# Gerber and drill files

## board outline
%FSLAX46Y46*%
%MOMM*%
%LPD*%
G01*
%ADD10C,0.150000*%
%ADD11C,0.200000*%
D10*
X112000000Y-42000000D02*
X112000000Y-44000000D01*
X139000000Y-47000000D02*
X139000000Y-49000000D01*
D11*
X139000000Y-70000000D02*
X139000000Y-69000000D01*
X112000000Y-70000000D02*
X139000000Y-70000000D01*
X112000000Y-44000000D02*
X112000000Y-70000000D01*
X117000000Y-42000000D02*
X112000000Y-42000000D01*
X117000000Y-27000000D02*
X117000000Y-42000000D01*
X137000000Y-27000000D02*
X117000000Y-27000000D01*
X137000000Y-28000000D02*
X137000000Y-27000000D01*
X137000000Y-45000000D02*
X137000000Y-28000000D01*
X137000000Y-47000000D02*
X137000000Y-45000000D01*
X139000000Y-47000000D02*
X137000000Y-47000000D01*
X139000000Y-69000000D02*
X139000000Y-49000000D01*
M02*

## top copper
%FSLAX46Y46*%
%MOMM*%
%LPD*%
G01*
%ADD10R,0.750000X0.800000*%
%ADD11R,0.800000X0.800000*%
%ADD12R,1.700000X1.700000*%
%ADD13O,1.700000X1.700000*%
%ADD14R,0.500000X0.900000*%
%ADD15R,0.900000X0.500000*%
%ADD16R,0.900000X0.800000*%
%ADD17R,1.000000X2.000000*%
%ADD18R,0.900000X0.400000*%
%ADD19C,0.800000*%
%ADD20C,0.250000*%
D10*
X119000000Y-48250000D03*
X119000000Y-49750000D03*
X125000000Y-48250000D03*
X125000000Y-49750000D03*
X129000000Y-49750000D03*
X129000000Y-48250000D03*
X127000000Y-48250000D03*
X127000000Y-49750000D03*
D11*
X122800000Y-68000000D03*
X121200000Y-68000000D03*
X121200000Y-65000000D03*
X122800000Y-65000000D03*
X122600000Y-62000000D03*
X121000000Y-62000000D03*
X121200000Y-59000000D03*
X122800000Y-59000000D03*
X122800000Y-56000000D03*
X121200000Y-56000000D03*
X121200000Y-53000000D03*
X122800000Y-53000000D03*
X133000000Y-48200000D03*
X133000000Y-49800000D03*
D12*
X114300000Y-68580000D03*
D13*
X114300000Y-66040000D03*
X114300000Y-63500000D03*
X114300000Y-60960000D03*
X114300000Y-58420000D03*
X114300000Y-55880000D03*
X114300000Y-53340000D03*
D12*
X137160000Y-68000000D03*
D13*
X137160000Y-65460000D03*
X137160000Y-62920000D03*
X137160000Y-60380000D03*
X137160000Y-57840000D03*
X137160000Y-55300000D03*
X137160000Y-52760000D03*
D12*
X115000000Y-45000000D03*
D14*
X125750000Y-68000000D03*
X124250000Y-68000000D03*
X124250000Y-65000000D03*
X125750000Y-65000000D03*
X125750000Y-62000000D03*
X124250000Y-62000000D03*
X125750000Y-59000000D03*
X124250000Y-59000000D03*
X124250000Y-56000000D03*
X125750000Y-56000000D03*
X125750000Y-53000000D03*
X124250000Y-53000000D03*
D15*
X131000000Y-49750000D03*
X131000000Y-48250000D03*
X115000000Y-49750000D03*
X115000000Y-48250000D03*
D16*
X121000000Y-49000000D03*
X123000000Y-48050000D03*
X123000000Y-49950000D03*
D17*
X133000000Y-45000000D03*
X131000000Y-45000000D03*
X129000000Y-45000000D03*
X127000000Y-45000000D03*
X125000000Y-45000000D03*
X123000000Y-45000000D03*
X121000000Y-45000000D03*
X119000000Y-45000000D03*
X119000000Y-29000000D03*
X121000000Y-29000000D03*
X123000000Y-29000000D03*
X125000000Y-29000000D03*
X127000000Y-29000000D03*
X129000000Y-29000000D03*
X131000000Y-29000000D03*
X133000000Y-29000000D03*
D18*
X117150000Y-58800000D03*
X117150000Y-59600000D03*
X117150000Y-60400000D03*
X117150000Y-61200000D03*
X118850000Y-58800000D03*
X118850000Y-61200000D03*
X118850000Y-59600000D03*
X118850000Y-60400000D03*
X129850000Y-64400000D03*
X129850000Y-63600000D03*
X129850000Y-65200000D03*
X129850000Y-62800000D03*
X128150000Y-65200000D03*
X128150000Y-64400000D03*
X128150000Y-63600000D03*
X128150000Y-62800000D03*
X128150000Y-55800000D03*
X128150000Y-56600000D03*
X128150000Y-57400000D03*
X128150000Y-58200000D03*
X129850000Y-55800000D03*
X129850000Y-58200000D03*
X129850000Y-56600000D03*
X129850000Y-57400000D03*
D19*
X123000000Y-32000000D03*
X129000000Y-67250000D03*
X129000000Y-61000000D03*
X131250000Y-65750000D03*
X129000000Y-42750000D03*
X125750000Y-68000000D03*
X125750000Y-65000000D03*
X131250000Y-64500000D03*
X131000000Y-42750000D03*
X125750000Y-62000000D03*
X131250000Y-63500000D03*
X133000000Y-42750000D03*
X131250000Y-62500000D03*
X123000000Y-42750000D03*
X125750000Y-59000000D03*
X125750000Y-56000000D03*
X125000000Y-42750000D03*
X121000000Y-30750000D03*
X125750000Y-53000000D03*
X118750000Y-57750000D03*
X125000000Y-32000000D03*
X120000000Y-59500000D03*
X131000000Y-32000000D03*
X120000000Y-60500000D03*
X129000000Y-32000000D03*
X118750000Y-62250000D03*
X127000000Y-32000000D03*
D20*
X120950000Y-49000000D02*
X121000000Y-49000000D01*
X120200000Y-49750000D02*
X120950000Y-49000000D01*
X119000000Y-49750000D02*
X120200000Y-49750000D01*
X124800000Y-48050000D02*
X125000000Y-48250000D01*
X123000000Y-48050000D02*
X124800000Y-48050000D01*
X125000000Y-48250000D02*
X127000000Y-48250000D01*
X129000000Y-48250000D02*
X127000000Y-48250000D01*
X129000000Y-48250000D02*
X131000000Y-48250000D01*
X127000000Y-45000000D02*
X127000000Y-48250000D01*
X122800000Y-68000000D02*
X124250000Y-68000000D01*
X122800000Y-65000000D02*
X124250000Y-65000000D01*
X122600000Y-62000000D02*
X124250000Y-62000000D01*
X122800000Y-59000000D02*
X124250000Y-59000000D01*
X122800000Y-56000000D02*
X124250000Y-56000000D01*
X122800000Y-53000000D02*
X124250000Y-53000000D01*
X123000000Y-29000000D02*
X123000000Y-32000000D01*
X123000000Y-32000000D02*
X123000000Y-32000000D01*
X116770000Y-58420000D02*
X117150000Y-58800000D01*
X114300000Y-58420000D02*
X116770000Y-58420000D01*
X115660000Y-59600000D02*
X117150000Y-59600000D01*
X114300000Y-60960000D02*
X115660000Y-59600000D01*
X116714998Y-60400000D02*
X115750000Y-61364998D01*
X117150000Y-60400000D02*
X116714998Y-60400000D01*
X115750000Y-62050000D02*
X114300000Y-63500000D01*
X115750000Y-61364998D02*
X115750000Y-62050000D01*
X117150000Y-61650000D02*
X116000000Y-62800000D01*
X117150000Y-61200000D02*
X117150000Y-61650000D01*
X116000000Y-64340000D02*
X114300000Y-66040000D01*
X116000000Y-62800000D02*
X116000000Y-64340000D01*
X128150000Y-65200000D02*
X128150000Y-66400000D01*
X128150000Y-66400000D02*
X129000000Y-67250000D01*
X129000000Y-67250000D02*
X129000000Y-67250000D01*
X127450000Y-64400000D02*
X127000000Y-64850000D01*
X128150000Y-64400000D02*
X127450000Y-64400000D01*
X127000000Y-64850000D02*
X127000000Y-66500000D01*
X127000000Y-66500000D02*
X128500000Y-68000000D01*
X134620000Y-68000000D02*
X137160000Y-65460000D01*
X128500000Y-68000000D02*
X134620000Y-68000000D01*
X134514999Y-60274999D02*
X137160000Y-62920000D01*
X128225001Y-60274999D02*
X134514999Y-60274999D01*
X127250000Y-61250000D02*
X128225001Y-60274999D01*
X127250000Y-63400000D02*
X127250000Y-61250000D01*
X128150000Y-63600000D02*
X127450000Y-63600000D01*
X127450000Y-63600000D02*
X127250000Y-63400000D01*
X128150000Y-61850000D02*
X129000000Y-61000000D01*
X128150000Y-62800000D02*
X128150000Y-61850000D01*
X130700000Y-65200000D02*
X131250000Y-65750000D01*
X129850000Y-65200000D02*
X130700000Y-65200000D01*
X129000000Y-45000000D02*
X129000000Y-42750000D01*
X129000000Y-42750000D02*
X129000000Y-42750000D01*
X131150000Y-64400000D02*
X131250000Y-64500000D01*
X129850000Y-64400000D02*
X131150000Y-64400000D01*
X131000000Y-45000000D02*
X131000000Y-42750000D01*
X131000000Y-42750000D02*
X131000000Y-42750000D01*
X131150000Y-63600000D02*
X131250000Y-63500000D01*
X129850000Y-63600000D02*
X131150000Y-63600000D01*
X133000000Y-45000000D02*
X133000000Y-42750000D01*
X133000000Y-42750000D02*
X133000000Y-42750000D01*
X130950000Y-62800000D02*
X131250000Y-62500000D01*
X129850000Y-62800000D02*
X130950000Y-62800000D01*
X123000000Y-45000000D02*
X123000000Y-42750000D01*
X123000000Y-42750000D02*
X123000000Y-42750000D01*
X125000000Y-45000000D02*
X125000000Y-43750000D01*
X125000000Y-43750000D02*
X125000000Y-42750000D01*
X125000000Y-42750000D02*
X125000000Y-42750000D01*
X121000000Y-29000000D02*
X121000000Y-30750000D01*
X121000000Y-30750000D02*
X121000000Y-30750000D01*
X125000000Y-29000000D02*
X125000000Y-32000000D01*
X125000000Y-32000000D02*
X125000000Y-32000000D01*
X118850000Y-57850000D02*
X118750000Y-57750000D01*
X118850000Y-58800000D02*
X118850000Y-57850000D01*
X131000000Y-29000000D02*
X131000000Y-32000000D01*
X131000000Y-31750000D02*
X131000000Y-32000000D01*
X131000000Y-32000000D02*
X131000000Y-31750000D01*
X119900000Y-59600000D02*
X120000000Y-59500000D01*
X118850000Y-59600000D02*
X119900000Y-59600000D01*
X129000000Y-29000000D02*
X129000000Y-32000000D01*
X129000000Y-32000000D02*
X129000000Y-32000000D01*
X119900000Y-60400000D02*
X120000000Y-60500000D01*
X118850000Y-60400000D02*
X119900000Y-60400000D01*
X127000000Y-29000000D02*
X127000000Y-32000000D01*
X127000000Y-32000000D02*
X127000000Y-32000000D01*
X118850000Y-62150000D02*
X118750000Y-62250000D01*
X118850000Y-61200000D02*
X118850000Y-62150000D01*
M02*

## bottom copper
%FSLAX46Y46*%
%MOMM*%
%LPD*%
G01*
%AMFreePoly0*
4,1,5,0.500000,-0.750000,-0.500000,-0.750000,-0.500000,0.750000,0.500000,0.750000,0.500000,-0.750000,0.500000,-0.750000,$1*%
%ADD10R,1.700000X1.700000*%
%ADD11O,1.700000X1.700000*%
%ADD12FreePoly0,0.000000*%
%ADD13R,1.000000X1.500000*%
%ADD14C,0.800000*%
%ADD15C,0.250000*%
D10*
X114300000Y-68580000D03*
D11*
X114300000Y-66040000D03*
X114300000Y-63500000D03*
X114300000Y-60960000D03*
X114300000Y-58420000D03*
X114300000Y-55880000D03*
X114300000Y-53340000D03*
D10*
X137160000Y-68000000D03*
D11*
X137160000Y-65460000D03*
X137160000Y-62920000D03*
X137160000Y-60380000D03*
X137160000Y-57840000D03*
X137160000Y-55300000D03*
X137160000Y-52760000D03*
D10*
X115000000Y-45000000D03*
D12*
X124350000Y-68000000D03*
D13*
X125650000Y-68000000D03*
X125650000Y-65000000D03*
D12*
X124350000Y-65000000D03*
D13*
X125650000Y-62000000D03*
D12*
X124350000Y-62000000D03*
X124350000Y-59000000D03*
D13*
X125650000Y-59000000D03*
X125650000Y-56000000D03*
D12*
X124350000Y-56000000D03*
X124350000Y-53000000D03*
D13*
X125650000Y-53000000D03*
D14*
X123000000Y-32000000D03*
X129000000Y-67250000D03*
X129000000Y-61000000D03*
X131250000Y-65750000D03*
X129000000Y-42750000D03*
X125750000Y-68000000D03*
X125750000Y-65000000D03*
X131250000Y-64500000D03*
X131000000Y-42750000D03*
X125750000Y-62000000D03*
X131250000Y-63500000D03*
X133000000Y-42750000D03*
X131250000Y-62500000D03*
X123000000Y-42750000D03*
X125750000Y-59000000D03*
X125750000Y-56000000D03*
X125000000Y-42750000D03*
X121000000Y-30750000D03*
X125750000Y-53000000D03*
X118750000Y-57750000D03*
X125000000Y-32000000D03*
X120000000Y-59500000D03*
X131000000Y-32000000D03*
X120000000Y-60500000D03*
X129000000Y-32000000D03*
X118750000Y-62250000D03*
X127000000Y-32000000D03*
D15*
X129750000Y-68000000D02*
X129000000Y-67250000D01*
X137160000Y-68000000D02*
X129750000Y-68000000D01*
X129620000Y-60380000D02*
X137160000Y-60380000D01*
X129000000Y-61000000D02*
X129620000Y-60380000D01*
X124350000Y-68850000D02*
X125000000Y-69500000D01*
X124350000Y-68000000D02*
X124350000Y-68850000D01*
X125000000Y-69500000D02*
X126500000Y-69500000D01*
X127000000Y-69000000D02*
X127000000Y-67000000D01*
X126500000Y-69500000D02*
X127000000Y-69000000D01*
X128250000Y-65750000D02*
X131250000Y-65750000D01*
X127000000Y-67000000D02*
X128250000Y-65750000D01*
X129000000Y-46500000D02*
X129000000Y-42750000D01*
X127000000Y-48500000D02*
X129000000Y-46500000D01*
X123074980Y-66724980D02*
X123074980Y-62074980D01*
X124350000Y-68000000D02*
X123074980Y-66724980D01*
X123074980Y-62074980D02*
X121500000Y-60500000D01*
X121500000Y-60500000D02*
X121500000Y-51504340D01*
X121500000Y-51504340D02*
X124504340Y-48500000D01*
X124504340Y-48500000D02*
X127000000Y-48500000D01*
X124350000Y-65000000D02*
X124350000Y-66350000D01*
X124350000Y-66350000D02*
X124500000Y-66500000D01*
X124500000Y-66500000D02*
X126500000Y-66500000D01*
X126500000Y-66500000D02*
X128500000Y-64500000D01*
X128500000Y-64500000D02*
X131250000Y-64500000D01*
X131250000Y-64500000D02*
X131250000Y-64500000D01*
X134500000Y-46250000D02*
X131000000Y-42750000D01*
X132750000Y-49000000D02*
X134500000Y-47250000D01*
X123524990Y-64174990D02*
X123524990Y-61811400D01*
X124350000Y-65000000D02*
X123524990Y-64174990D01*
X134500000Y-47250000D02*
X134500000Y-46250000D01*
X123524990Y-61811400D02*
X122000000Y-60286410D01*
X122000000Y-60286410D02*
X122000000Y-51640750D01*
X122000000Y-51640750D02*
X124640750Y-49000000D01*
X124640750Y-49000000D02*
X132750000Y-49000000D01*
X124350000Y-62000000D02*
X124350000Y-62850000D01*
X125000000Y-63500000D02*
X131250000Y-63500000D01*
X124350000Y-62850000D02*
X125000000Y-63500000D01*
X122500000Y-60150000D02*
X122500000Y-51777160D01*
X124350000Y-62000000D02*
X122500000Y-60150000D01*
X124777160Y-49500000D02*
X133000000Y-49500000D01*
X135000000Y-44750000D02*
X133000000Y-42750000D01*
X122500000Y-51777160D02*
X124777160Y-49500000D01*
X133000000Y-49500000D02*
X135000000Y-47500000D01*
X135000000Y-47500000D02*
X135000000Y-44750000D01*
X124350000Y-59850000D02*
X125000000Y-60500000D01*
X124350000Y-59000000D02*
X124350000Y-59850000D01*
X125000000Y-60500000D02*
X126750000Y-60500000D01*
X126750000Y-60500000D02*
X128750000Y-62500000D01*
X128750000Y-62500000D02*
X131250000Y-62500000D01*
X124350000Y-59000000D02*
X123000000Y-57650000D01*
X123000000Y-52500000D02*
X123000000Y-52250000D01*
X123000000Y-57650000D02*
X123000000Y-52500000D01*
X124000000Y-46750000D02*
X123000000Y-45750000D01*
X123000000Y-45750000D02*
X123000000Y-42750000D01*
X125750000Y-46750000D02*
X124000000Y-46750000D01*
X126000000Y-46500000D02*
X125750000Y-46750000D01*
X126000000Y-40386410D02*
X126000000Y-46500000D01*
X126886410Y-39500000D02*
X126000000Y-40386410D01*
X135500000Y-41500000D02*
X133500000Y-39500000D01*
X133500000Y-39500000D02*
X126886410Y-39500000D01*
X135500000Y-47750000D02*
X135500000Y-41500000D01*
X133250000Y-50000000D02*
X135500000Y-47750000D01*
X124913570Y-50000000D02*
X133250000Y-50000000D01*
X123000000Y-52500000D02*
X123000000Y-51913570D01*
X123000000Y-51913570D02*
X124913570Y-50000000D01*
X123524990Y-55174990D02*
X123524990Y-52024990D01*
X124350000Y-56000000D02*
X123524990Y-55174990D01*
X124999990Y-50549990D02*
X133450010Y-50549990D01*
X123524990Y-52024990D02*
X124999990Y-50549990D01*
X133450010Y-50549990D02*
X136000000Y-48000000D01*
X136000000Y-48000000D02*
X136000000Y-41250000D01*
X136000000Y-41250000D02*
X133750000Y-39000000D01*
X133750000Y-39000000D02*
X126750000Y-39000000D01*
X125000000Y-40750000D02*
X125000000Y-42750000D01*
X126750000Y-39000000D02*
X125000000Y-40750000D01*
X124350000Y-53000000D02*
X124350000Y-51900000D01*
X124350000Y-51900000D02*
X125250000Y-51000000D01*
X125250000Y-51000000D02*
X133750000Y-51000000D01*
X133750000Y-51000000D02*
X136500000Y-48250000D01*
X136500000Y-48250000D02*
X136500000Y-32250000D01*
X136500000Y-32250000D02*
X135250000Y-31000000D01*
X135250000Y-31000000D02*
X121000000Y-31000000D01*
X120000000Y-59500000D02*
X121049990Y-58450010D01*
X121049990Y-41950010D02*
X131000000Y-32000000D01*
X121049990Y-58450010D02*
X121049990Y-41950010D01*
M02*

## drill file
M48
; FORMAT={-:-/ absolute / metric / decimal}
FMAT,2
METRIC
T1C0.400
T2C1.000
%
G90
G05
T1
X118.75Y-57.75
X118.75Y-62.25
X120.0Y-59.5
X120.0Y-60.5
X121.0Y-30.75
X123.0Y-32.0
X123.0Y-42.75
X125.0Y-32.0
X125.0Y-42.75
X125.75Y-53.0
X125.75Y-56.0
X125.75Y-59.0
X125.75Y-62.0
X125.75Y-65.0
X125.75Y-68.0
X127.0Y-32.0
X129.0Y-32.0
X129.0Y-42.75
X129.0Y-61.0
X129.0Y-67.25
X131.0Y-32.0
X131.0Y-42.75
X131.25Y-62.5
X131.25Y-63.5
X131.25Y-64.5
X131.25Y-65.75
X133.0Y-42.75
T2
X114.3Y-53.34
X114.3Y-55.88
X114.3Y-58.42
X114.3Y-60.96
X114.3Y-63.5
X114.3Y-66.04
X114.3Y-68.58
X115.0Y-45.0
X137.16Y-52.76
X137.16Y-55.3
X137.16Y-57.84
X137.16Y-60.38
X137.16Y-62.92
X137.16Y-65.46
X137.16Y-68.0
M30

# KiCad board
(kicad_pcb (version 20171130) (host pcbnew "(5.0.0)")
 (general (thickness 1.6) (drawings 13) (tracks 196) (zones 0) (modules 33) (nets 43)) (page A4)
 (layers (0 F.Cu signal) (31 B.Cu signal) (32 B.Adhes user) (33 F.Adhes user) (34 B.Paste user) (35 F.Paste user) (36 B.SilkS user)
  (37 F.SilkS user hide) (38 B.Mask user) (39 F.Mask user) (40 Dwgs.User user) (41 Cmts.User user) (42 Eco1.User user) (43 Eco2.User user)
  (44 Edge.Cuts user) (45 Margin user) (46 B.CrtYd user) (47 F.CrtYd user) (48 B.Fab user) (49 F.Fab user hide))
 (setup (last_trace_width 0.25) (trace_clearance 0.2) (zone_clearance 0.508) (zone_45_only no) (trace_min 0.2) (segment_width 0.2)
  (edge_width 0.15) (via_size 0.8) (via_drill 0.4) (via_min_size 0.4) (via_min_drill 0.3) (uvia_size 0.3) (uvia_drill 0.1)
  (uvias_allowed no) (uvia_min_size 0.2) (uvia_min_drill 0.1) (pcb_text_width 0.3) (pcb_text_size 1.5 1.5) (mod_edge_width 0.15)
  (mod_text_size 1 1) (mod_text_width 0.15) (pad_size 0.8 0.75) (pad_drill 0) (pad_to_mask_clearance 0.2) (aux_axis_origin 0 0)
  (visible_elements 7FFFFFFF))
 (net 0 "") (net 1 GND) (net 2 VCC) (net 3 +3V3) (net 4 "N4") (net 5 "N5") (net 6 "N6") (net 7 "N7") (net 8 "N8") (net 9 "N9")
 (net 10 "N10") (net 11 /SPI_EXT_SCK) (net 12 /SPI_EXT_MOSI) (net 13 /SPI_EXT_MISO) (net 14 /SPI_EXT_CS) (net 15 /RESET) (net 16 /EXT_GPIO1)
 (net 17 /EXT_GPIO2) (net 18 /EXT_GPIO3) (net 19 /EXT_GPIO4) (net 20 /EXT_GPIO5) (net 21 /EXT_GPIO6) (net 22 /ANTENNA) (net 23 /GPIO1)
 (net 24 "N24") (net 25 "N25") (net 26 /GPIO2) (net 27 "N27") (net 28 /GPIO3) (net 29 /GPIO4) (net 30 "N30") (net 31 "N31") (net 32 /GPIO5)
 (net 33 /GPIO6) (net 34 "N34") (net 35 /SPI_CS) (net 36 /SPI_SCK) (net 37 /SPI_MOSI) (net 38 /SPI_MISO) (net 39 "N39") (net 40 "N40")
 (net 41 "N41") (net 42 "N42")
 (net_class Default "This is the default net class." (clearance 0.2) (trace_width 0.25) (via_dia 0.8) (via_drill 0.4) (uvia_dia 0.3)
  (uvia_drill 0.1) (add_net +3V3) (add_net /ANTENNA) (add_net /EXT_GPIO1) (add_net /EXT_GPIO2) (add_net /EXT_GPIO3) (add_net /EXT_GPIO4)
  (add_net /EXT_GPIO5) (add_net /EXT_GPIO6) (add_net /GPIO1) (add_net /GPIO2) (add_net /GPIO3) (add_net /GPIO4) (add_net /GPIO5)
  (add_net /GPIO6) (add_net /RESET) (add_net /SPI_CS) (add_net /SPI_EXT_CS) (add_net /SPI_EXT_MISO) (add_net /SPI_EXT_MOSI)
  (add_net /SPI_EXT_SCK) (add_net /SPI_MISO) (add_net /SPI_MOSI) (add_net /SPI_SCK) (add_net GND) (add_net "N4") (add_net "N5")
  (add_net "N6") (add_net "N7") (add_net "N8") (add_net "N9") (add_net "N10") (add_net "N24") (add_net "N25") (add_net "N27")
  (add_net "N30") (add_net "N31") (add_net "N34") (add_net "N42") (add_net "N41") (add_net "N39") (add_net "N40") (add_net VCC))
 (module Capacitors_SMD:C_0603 (layer F.Cu) (at 119 49 90)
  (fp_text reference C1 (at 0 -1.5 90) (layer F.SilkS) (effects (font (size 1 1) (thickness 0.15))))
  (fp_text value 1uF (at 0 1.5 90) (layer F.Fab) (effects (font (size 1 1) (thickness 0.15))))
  (pad 2 smd rect (at 0.75 0 90) (size 0.8 0.75) (layers F.Cu F.Paste F.Mask) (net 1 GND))
  (pad 1 smd rect (at -0.75 0 90) (size 0.8 0.75) (layers F.Cu F.Paste F.Mask) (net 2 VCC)))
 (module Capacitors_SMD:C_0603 (layer F.Cu) (at 125 49 270)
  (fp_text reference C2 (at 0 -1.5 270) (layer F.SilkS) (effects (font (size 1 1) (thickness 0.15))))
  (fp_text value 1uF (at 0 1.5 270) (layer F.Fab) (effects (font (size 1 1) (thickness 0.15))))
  (pad 1 smd rect (at -0.75 0 270) (size 0.8 0.75) (layers F.Cu F.Paste F.Mask) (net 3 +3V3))
  (pad 2 smd rect (at 0.75 0 270) (size 0.8 0.75) (layers F.Cu F.Paste F.Mask) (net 1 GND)))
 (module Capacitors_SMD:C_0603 (layer F.Cu) (at 129 49 270)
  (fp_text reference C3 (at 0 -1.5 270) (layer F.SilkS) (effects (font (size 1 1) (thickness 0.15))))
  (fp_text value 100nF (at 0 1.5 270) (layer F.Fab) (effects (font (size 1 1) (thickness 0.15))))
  (pad 2 smd rect (at 0.75 0 270) (size 0.8 0.75) (layers F.Cu F.Paste F.Mask) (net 1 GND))
  (pad 1 smd rect (at -0.75 0 270) (size 0.8 0.75) (layers F.Cu F.Paste F.Mask) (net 3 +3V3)))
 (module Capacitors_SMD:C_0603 (layer F.Cu) (at 127 49 270)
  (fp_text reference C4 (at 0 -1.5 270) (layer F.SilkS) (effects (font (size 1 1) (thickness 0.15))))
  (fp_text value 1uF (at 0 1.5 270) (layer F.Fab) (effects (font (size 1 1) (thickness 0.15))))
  (pad 1 smd rect (at -0.75 0 270) (size 0.8 0.75) (layers F.Cu F.Paste F.Mask) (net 3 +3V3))
  (pad 2 smd rect (at 0.75 0 270) (size 0.8 0.75) (layers F.Cu F.Paste F.Mask) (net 1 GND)))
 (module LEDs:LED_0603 (layer F.Cu) (at 122 68)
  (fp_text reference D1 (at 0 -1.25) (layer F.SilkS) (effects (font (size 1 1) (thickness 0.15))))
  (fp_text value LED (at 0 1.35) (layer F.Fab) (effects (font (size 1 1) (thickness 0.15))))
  (pad 2 smd rect (at 0.8 0 180) (size 0.8 0.8) (layers F.Cu F.Paste F.Mask) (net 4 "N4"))
  (pad 1 smd rect (at -0.8 0 180) (size 0.8 0.8) (layers F.Cu F.Paste F.Mask) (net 1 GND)))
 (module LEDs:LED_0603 (layer F.Cu) (at 122 65)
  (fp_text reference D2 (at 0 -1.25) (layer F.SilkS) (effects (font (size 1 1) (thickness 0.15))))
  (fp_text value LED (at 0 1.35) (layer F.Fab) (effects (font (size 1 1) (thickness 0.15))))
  (pad 1 smd rect (at -0.8 0 180) (size 0.8 0.8) (layers F.Cu F.Paste F.Mask) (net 1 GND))
  (pad 2 smd rect (at 0.8 0 180) (size 0.8 0.8) (layers F.Cu F.Paste F.Mask) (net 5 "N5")))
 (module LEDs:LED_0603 (layer F.Cu) (at 121.8 62)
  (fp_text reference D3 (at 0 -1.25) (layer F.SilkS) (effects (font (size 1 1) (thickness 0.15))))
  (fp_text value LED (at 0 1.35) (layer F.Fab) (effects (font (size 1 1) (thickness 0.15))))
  (pad 2 smd rect (at 0.8 0 180) (size 0.8 0.8) (layers F.Cu F.Paste F.Mask) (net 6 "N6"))
  (pad 1 smd rect (at -0.8 0 180) (size 0.8 0.8) (layers F.Cu F.Paste F.Mask) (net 1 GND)))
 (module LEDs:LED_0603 (layer F.Cu) (at 122 59)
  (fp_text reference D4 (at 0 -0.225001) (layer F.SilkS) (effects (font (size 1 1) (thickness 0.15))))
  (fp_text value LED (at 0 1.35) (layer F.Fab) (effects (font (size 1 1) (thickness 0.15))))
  (pad 1 smd rect (at -0.8 0 180) (size 0.8 0.8) (layers F.Cu F.Paste F.Mask) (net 1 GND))
  (pad 2 smd rect (at 0.8 0 180) (size 0.8 0.8) (layers F.Cu F.Paste F.Mask) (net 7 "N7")))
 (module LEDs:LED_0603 (layer F.Cu) (at 122 56)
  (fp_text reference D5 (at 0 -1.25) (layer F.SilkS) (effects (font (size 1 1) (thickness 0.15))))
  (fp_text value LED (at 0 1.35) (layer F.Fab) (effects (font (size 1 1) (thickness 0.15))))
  (pad 2 smd rect (at 0.8 0 180) (size 0.8 0.8) (layers F.Cu F.Paste F.Mask) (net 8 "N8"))
  (pad 1 smd rect (at -0.8 0 180) (size 0.8 0.8) (layers F.Cu F.Paste F.Mask) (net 1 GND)))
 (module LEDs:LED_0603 (layer F.Cu) (at 122 53)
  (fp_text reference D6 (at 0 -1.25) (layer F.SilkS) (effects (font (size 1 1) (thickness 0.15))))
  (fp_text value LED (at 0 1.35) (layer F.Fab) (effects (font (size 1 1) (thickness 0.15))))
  (pad 1 smd rect (at -0.8 0 180) (size 0.8 0.8) (layers F.Cu F.Paste F.Mask) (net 1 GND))
  (pad 2 smd rect (at 0.8 0 180) (size 0.8 0.8) (layers F.Cu F.Paste F.Mask) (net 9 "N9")))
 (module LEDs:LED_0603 (layer F.Cu) (at 133 49 270)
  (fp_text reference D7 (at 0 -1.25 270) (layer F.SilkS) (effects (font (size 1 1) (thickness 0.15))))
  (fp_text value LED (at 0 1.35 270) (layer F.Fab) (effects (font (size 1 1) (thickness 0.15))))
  (pad 1 smd rect (at -0.8 0 90) (size 0.8 0.8) (layers F.Cu F.Paste F.Mask) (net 1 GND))
  (pad 2 smd rect (at 0.8 0 90) (size 0.8 0.8) (layers F.Cu F.Paste F.Mask) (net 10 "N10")))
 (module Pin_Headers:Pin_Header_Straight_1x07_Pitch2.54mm (layer F.Cu) (at 114.3 68.58 180)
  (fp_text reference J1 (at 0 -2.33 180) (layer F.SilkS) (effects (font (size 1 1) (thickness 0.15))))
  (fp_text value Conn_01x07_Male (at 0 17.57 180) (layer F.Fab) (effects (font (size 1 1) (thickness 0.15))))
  (pad 1 thru_hole rect (at 0 0 180) (size 1.7 1.7) (drill 1) (layers *.Cu *.Mask) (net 2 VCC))
  (pad 2 thru_hole oval (at 0 2.54 180) (size 1.7 1.7) (drill 1) (layers *.Cu *.Mask) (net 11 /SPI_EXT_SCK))
  (pad 3 thru_hole oval (at 0 5.08 180) (size 1.7 1.7) (drill 1) (layers *.Cu *.Mask) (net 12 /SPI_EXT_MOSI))
  (pad 4 thru_hole oval (at 0 7.62 180) (size 1.7 1.7) (drill 1) (layers *.Cu *.Mask) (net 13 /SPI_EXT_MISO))
  (pad 5 thru_hole oval (at 0 10.16 180) (size 1.7 1.7) (drill 1) (layers *.Cu *.Mask) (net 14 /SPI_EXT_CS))
  (pad 6 thru_hole oval (at 0 12.7 180) (size 1.7 1.7) (drill 1) (layers *.Cu *.Mask) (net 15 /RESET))
  (pad 7 thru_hole oval (at 0 15.24 180) (size 1.7 1.7) (drill 1) (layers *.Cu *.Mask) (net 1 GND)))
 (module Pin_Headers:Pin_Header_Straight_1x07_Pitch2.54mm (layer F.Cu) (at 137.16 68 180)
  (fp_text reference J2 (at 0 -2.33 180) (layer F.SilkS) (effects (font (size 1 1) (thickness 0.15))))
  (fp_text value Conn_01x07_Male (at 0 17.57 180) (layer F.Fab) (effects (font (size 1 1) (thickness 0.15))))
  (pad 1 thru_hole rect (at 0 0 180) (size 1.7 1.7) (drill 1) (layers *.Cu *.Mask) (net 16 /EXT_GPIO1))
  (pad 2 thru_hole oval (at 0 2.54 180) (size 1.7 1.7) (drill 1) (layers *.Cu *.Mask) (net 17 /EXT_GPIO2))
  (pad 3 thru_hole oval (at 0 5.08 180) (size 1.7 1.7) (drill 1) (layers *.Cu *.Mask) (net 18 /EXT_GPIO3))
  (pad 4 thru_hole oval (at 0 7.62 180) (size 1.7 1.7) (drill 1) (layers *.Cu *.Mask) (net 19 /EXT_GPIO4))
  (pad 5 thru_hole oval (at 0 10.16 180) (size 1.7 1.7) (drill 1) (layers *.Cu *.Mask) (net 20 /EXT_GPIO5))
  (pad 6 thru_hole oval (at 0 12.7 180) (size 1.7 1.7) (drill 1) (layers *.Cu *.Mask) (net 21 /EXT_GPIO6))
  (pad 7 thru_hole oval (at 0 15.24 180) (size 1.7 1.7) (drill 1) (layers *.Cu *.Mask) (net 1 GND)))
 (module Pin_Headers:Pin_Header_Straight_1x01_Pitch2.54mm (layer F.Cu) (at 115 45)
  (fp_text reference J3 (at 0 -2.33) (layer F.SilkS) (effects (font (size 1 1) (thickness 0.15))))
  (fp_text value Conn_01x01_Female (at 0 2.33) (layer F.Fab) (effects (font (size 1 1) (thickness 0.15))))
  (pad 1 thru_hole rect (at 0 0) (size 1.7 1.7) (drill 1) (layers *.Cu *.Mask) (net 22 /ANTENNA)))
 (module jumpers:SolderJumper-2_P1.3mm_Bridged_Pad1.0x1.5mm (layer B.Cu) (at 125 68)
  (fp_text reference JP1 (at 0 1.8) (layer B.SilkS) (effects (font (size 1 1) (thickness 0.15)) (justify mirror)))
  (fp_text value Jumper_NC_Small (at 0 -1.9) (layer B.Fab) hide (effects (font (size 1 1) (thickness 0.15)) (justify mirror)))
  (pad 1 smd custom (at -0.65 0) (size 1 1.5) (layers B.Cu B.Mask) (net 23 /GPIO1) (options (clearance outline) (anchor rect)) (primitives))
  (pad 2 smd rect (at 0.65 0) (size 1 1.5) (layers B.Cu B.Mask) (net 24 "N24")))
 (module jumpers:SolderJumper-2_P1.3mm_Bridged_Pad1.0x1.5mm (layer B.Cu) (at 125 65)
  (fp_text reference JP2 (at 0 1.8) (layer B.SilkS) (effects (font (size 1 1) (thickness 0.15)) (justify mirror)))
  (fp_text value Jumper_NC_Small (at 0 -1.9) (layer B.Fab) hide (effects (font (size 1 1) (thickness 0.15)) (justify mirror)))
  (pad 2 smd rect (at 0.65 0) (size 1 1.5) (layers B.Cu B.Mask) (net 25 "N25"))
  (pad 1 smd custom (at -0.65 0) (size 1 1.5) (layers B.Cu B.Mask) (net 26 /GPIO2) (options (clearance outline) (anchor rect)) (primitives)))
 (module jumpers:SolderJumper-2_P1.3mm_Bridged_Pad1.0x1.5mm (layer B.Cu) (at 125 62)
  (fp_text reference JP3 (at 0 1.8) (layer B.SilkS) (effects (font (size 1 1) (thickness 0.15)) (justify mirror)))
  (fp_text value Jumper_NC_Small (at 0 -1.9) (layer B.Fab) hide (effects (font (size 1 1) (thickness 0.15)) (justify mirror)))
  (pad 2 smd rect (at 0.65 0) (size 1 1.5) (layers B.Cu B.Mask) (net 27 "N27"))
  (pad 1 smd custom (at -0.65 0) (size 1 1.5) (layers B.Cu B.Mask) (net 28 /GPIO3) (options (clearance outline) (anchor rect)) (primitives)))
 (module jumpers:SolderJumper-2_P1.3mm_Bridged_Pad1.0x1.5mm (layer B.Cu) (at 125 59)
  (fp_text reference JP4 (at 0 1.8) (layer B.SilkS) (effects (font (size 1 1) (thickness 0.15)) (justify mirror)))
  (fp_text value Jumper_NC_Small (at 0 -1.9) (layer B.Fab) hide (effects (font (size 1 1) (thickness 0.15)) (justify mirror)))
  (pad 1 smd custom (at -0.65 0) (size 1 1.5) (layers B.Cu B.Mask) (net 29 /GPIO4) (options (clearance outline) (anchor rect)) (primitives))
  (pad 2 smd rect (at 0.65 0) (size 1 1.5) (layers B.Cu B.Mask) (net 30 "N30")))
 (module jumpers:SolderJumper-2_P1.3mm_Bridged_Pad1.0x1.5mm (layer B.Cu) (at 125 56)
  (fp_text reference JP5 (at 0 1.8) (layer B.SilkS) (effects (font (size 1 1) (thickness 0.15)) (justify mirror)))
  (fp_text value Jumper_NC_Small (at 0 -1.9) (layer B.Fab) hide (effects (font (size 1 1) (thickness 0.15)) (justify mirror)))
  (pad 2 smd rect (at 0.65 0) (size 1 1.5) (layers B.Cu B.Mask) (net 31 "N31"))
  (pad 1 smd custom (at -0.65 0) (size 1 1.5) (layers B.Cu B.Mask) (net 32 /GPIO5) (options (clearance outline) (anchor rect)) (primitives)))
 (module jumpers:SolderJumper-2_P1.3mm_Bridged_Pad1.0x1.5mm (layer B.Cu) (at 125 53)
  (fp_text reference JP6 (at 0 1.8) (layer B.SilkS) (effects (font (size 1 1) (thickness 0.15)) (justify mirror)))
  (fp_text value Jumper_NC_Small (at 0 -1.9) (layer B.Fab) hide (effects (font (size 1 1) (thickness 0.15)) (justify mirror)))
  (pad 1 smd custom (at -0.65 0) (size 1 1.5) (layers B.Cu B.Mask) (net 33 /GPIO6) (options (clearance outline) (anchor rect)) (primitives))
  (pad 2 smd rect (at 0.65 0) (size 1 1.5) (layers B.Cu B.Mask) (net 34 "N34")))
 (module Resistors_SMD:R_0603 (layer F.Cu) (at 125 68)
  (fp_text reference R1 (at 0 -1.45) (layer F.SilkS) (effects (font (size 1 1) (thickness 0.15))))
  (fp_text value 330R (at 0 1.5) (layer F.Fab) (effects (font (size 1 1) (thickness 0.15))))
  (pad 2 smd rect (at 0.75 0) (size 0.5 0.9) (layers F.Cu F.Paste F.Mask) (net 24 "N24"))
  (pad 1 smd rect (at -0.75 0) (size 0.5 0.9) (layers F.Cu F.Paste F.Mask) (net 4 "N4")))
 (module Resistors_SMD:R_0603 (layer F.Cu) (at 125 65)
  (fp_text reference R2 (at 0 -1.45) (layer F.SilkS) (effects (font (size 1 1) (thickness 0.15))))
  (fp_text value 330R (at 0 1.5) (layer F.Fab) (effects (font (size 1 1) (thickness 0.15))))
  (pad 1 smd rect (at -0.75 0) (size 0.5 0.9) (layers F.Cu F.Paste F.Mask) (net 5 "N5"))
  (pad 2 smd rect (at 0.75 0) (size 0.5 0.9) (layers F.Cu F.Paste F.Mask) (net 25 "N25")))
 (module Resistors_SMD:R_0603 (layer F.Cu) (at 125 62)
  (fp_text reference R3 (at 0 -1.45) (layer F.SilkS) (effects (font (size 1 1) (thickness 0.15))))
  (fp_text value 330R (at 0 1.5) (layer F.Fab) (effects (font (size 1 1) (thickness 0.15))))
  (pad 2 smd rect (at 0.75 0) (size 0.5 0.9) (layers F.Cu F.Paste F.Mask) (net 27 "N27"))
  (pad 1 smd rect (at -0.75 0) (size 0.5 0.9) (layers F.Cu F.Paste F.Mask) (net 6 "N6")))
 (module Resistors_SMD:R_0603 (layer F.Cu) (at 125 59)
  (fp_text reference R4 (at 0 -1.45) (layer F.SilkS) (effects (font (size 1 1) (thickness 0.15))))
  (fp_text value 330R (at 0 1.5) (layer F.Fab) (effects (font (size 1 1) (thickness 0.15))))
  (pad 2 smd rect (at 0.75 0) (size 0.5 0.9) (layers F.Cu F.Paste F.Mask) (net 30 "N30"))
  (pad 1 smd rect (at -0.75 0) (size 0.5 0.9) (layers F.Cu F.Paste F.Mask) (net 7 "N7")))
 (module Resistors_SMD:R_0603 (layer F.Cu) (at 125 56)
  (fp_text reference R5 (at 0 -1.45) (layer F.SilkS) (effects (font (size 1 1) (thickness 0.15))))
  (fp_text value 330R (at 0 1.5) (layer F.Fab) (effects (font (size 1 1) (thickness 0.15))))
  (pad 1 smd rect (at -0.75 0) (size 0.5 0.9) (layers F.Cu F.Paste F.Mask) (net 8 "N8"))
  (pad 2 smd rect (at 0.75 0) (size 0.5 0.9) (layers F.Cu F.Paste F.Mask) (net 31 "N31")))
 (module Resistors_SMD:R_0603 (layer F.Cu) (at 125 53)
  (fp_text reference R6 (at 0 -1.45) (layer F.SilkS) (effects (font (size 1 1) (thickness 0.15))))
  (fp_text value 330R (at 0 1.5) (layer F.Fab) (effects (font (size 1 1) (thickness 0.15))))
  (pad 2 smd rect (at 0.75 0) (size 0.5 0.9) (layers F.Cu F.Paste F.Mask) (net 34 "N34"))
  (pad 1 smd rect (at -0.75 0) (size 0.5 0.9) (layers F.Cu F.Paste F.Mask) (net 9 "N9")))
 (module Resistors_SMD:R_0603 (layer F.Cu) (at 131 49 90)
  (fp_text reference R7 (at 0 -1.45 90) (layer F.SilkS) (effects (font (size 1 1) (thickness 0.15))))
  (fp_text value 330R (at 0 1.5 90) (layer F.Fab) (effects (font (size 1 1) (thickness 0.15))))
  (pad 1 smd rect (at -0.75 0 90) (size 0.5 0.9) (layers F.Cu F.Paste F.Mask) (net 10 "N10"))
  (pad 2 smd rect (at 0.75 0 90) (size 0.5 0.9) (layers F.Cu F.Paste F.Mask) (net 3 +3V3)))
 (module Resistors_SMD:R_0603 (layer F.Cu) (at 115 49 90)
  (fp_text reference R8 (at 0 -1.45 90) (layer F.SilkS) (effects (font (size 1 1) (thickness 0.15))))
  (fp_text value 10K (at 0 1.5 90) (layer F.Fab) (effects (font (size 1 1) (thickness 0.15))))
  (pad 1 smd rect (at -0.75 0 90) (size 0.5 0.9) (layers F.Cu F.Paste F.Mask) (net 15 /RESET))
  (pad 2 smd rect (at 0.75 0 90) (size 0.5 0.9) (layers F.Cu F.Paste F.Mask) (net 3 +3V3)))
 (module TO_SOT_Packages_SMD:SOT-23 (layer F.Cu) (at 122 49 180)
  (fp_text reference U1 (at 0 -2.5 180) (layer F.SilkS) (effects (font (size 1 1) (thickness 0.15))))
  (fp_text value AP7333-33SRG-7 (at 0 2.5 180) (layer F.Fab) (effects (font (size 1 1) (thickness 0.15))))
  (pad 3 smd rect (at 1 0 180) (size 0.9 0.8) (layers F.Cu F.Paste F.Mask) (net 2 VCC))
  (pad 2 smd rect (at -1 0.95 180) (size 0.9 0.8) (layers F.Cu F.Paste F.Mask) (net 3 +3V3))
  (pad 1 smd rect (at -1 -0.95 180) (size 0.9 0.8) (layers F.Cu F.Paste F.Mask) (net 1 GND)))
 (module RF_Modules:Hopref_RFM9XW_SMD (layer F.Cu) (at 126 37 270)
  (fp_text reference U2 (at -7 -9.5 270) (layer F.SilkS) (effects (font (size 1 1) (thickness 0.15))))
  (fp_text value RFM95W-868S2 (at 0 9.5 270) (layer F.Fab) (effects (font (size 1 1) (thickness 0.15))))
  (pad 16 smd rect (at 8 -7 270) (size 2 1) (layers F.Cu F.Paste F.Mask) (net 28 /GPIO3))
  (pad 15 smd rect (at 8 -5 270) (size 2 1) (layers F.Cu F.Paste F.Mask) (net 26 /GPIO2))
  (pad 14 smd rect (at 8 -3 270) (size 2 1) (layers F.Cu F.Paste F.Mask) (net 23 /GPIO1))
  (pad 13 smd rect (at 8 -1 270) (size 2 1) (layers F.Cu F.Paste F.Mask) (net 3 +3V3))
  (pad 12 smd rect (at 8 1 270) (size 2 1) (layers F.Cu F.Paste F.Mask) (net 32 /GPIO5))
  (pad 11 smd rect (at 8 3 270) (size 2 1) (layers F.Cu F.Paste F.Mask) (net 29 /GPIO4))
  (pad 10 smd rect (at 8 5 270) (size 2 1) (layers F.Cu F.Paste F.Mask) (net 1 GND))
  (pad 9 smd rect (at 8 7 270) (size 2 1) (layers F.Cu F.Paste F.Mask) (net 22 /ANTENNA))
  (pad 8 smd rect (at -8 7 270) (size 2 1) (layers F.Cu F.Paste F.Mask) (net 1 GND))
  (pad 7 smd rect (at -8 5 270) (size 2 1) (layers F.Cu F.Paste F.Mask) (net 33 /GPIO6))
  (pad 6 smd rect (at -8 3 270) (size 2 1) (layers F.Cu F.Paste F.Mask) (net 15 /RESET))
  (pad 5 smd rect (at -8 1 270) (size 2 1) (layers F.Cu F.Paste F.Mask) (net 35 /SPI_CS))
  (pad 4 smd rect (at -8 -1 270) (size 2 1) (layers F.Cu F.Paste F.Mask) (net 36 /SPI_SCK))
  (pad 3 smd rect (at -8 -3 270) (size 2 1) (layers F.Cu F.Paste F.Mask) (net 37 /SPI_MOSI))
  (pad 2 smd rect (at -8 -5 270) (size 2 1) (layers F.Cu F.Paste F.Mask) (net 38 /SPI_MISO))
  (pad 1 smd rect (at -8 -7 270) (size 2 1) (layers F.Cu F.Paste F.Mask) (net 1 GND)))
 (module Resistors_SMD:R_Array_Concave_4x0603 (layer F.Cu) (at 118 60 180)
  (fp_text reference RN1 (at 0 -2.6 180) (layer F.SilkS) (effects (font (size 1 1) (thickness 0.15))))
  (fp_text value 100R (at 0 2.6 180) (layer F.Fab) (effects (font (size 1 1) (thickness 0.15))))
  (pad 5 smd rect (at 0.85 1.2 180) (size 0.9 0.4) (layers F.Cu F.Paste F.Mask) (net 14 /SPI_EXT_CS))
  (pad 6 smd rect (at 0.85 0.4 180) (size 0.9 0.4) (layers F.Cu F.Paste F.Mask) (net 13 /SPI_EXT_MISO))
  (pad 7 smd rect (at 0.85 -0.4 180) (size 0.9 0.4) (layers F.Cu F.Paste F.Mask) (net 12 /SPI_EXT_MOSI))
  (pad 8 smd rect (at 0.85 -1.2 180) (size 0.9 0.4) (layers F.Cu F.Paste F.Mask) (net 11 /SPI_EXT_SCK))
  (pad 4 smd rect (at -0.85 1.2 180) (size 0.9 0.4) (layers F.Cu F.Paste F.Mask) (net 35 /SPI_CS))
  (pad 1 smd rect (at -0.85 -1.2 180) (size 0.9 0.4) (layers F.Cu F.Paste F.Mask) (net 36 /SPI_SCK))
  (pad 3 smd rect (at -0.85 0.4 180) (size 0.9 0.4) (layers F.Cu F.Paste F.Mask) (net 38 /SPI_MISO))
  (pad 2 smd rect (at -0.85 -0.4 180) (size 0.9 0.4) (layers F.Cu F.Paste F.Mask) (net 37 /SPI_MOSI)))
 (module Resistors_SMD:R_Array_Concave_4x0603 (layer F.Cu) (at 129 64 180)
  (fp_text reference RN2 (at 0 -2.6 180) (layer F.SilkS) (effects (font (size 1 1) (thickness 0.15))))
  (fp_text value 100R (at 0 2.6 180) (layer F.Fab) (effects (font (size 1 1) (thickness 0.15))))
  (pad 2 smd rect (at -0.85 -0.4 180) (size 0.9 0.4) (layers F.Cu F.Paste F.Mask) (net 26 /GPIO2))
  (pad 3 smd rect (at -0.85 0.4 180) (size 0.9 0.4) (layers F.Cu F.Paste F.Mask) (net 28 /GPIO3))
  (pad 1 smd rect (at -0.85 -1.2 180) (size 0.9 0.4) (layers F.Cu F.Paste F.Mask) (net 23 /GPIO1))
  (pad 4 smd rect (at -0.85 1.2 180) (size 0.9 0.4) (layers F.Cu F.Paste F.Mask) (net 29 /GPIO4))
  (pad 8 smd rect (at 0.85 -1.2 180) (size 0.9 0.4) (layers F.Cu F.Paste F.Mask) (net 16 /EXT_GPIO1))
  (pad 7 smd rect (at 0.85 -0.4 180) (size 0.9 0.4) (layers F.Cu F.Paste F.Mask) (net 17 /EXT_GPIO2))
  (pad 6 smd rect (at 0.85 0.4 180) (size 0.9 0.4) (layers F.Cu F.Paste F.Mask) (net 18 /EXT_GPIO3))
  (pad 5 smd rect (at 0.85 1.2 180) (size 0.9 0.4) (layers F.Cu F.Paste F.Mask) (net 19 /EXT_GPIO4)))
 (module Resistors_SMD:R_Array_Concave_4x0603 (layer F.Cu) (at 129 57 180)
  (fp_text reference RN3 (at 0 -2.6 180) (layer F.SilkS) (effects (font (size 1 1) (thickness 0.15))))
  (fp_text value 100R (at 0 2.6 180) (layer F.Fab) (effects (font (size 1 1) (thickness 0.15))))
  (pad 5 smd rect (at 0.85 1.2 180) (size 0.9 0.4) (layers F.Cu F.Paste F.Mask) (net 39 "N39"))
  (pad 6 smd rect (at 0.85 0.4 180) (size 0.9 0.4) (layers F.Cu F.Paste F.Mask) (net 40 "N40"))
  (pad 7 smd rect (at 0.85 -0.4 180) (size 0.9 0.4) (layers F.Cu F.Paste F.Mask) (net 21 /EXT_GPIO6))
  (pad 8 smd rect (at 0.85 -1.2 180) (size 0.9 0.4) (layers F.Cu F.Paste F.Mask) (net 20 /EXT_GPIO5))
  (pad 4 smd rect (at -0.85 1.2 180) (size 0.9 0.4) (layers F.Cu F.Paste F.Mask) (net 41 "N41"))
  (pad 1 smd rect (at -0.85 -1.2 180) (size 0.9 0.4) (layers F.Cu F.Paste F.Mask) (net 32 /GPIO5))
  (pad 3 smd rect (at -0.85 0.4 180) (size 0.9 0.4) (layers F.Cu F.Paste F.Mask) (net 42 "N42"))
  (pad 2 smd rect (at -0.85 -0.4 180) (size 0.9 0.4) (layers F.Cu F.Paste F.Mask) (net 33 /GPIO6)))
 (gr_line (start 112 42) (end 112 44) (layer Edge.Cuts) (width 0.15))
 (gr_line (start 139 47) (end 139 49) (layer Edge.Cuts) (width 0.15))
 (gr_line (start 139 70) (end 139 69) (layer Edge.Cuts) (width 0.2))
 (gr_line (start 112 70) (end 139 70) (layer Edge.Cuts) (width 0.2))
 (gr_line (start 112 44) (end 112 70) (layer Edge.Cuts) (width 0.2))
 (gr_line (start 117 42) (end 112 42) (layer Edge.Cuts) (width 0.2))
 (gr_line (start 117 27) (end 117 42) (layer Edge.Cuts) (width 0.2))
 (gr_line (start 137 27) (end 117 27) (layer Edge.Cuts) (width 0.2))
 (gr_line (start 137 28) (end 137 27) (layer Edge.Cuts) (width 0.2))
 (gr_line (start 137 45) (end 137 28) (layer Edge.Cuts) (width 0.2))
 (gr_line (start 137 47) (end 137 45) (layer Edge.Cuts) (width 0.2))
 (gr_line (start 139 47) (end 137 47) (layer Edge.Cuts) (width 0.2))
 (gr_line (start 139 69) (end 139 49) (layer Edge.Cuts) (width 0.2))
 (segment (start 120.95 49) (end 121 49) (width 0.25) (layer F.Cu) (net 2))
 (segment (start 120.2 49.75) (end 120.95 49) (width 0.25) (layer F.Cu) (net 2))
 (segment (start 119 49.75) (end 120.2 49.75) (width 0.25) (layer F.Cu) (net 2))
 (segment (start 124.8 48.05) (end 125 48.25) (width 0.25) (layer F.Cu) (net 3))
 (segment (start 123 48.05) (end 124.8 48.05) (width 0.25) (layer F.Cu) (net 3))
 (segment (start 125 48.25) (end 127 48.25) (width 0.25) (layer F.Cu) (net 3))
 (segment (start 129 48.25) (end 127 48.25) (width 0.25) (layer F.Cu) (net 3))
 (segment (start 129 48.25) (end 131 48.25) (width 0.25) (layer F.Cu) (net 3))
 (segment (start 127 45) (end 127 48.25) (width 0.25) (layer F.Cu) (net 3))
 (segment (start 122.8 68) (end 124.25 68) (width 0.25) (layer F.Cu) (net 4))
 (segment (start 122.8 65) (end 124.25 65) (width 0.25) (layer F.Cu) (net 5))
 (segment (start 122.6 62) (end 124.25 62) (width 0.25) (layer F.Cu) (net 6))
 (segment (start 122.8 59) (end 124.25 59) (width 0.25) (layer F.Cu) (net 7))
 (segment (start 122.8 56) (end 124.25 56) (width 0.25) (layer F.Cu) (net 8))
 (segment (start 122.8 53) (end 124.25 53) (width 0.25) (layer F.Cu) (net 9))
 (segment (start 123 29) (end 123 32) (width 0.25) (layer F.Cu) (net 15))
 (segment (start 123 32) (end 123 32) (width 0.25) (layer F.Cu) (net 15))
 (via (at 123 32) (size 0.8) (drill 0.4) (layers F.Cu B.Cu) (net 15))
 (segment (start 116.77 58.42) (end 117.15 58.8) (width 0.25) (layer F.Cu) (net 14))
 (segment (start 114.3 58.42) (end 116.77 58.42) (width 0.25) (layer F.Cu) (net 14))
 (segment (start 115.66 59.6) (end 117.15 59.6) (width 0.25) (layer F.Cu) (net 13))
 (segment (start 114.3 60.96) (end 115.66 59.6) (width 0.25) (layer F.Cu) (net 13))
 (segment (start 116.714998 60.4) (end 115.75 61.364998) (width 0.25) (layer F.Cu) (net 12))
 (segment (start 117.15 60.4) (end 116.714998 60.4) (width 0.25) (layer F.Cu) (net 12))
 (segment (start 115.75 62.05) (end 114.3 63.5) (width 0.25) (layer F.Cu) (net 12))
 (segment (start 115.75 61.364998) (end 115.75 62.05) (width 0.25) (layer F.Cu) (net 12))
 (segment (start 117.15 61.65) (end 116 62.8) (width 0.25) (layer F.Cu) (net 11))
 (segment (start 117.15 61.2) (end 117.15 61.65) (width 0.25) (layer F.Cu) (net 11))
 (segment (start 116 64.34) (end 114.3 66.04) (width 0.25) (layer F.Cu) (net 11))
 (segment (start 116 62.8) (end 116 64.34) (width 0.25) (layer F.Cu) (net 11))
 (segment (start 128.15 65.2) (end 128.15 66.4) (width 0.25) (layer F.Cu) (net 16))
 (segment (start 128.15 66.4) (end 129 67.25) (width 0.25) (layer F.Cu) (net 16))
 (segment (start 129 67.25) (end 129 67.25) (width 0.25) (layer F.Cu) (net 16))
 (via (at 129 67.25) (size 0.8) (drill 0.4) (layers F.Cu B.Cu) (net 16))
 (segment (start 129.75 68) (end 129 67.25) (width 0.25) (layer B.Cu) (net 16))
 (segment (start 137.16 68) (end 129.75 68) (width 0.25) (layer B.Cu) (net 16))
 (segment (start 127.45 64.4) (end 127 64.85) (width 0.25) (layer F.Cu) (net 17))
 (segment (start 128.15 64.4) (end 127.45 64.4) (width 0.25) (layer F.Cu) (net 17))
 (segment (start 127 64.85) (end 127 66.5) (width 0.25) (layer F.Cu) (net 17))
 (segment (start 127 66.5) (end 128.5 68) (width 0.25) (layer F.Cu) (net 17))
 (segment (start 134.62 68) (end 137.16 65.46) (width 0.25) (layer F.Cu) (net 17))
 (segment (start 128.5 68) (end 134.62 68) (width 0.25) (layer F.Cu) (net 17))
 (segment (start 134.514999 60.274999) (end 137.16 62.92) (width 0.25) (layer F.Cu) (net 18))
 (segment (start 128.225001 60.274999) (end 134.514999 60.274999) (width 0.25) (layer F.Cu) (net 18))
 (segment (start 127.25 61.25) (end 128.225001 60.274999) (width 0.25) (layer F.Cu) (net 18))
 (segment (start 127.25 63.4) (end 127.25 61.25) (width 0.25) (layer F.Cu) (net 18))
 (segment (start 128.15 63.6) (end 127.45 63.6) (width 0.25) (layer F.Cu) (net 18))
 (segment (start 127.45 63.6) (end 127.25 63.4) (width 0.25) (layer F.Cu) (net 18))
 (via (at 129 61) (size 0.8) (drill 0.4) (layers F.Cu B.Cu) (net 19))
 (segment (start 128.15 61.85) (end 129 61) (width 0.25) (layer F.Cu) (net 19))
 (segment (start 128.15 62.8) (end 128.15 61.85) (width 0.25) (layer F.Cu) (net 19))
 (segment (start 129.62 60.38) (end 137.16 60.38) (width 0.25) (layer B.Cu) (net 19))
 (segment (start 129 61) (end 129.62 60.38) (width 0.25) (layer B.Cu) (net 19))
 (via (at 131.25 65.75) (size 0.8) (drill 0.4) (layers F.Cu B.Cu) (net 23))
 (segment (start 124.35 68.85) (end 125 69.5) (width 0.25) (layer B.Cu) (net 23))
 (segment (start 124.35 68) (end 124.35 68.85) (width 0.25) (layer B.Cu) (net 23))
 (segment (start 125 69.5) (end 126.5 69.5) (width 0.25) (layer B.Cu) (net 23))
 (segment (start 127 69) (end 127 67) (width 0.25) (layer B.Cu) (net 23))
 (segment (start 126.5 69.5) (end 127 69) (width 0.25) (layer B.Cu) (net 23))
 (segment (start 128.25 65.75) (end 131.25 65.75) (width 0.25) (layer B.Cu) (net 23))
 (segment (start 127 67) (end 128.25 65.75) (width 0.25) (layer B.Cu) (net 23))
 (segment (start 130.7 65.2) (end 131.25 65.75) (width 0.25) (layer F.Cu) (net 23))
 (segment (start 129.85 65.2) (end 130.7 65.2) (width 0.25) (layer F.Cu) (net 23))
 (segment (start 129 45) (end 129 42.75) (width 0.25) (layer F.Cu) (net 23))
 (segment (start 129 42.75) (end 129 42.75) (width 0.25) (layer F.Cu) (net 23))
 (via (at 129 42.75) (size 0.8) (drill 0.4) (layers F.Cu B.Cu) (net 23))
 (segment (start 129 46.5) (end 129 42.75) (width 0.25) (layer B.Cu) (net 23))
 (segment (start 127 48.5) (end 129 46.5) (width 0.25) (layer B.Cu) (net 23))
 (segment (start 123.07498 66.72498) (end 123.07498 62.07498) (width 0.25) (layer B.Cu) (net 23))
 (segment (start 124.35 68) (end 123.07498 66.72498) (width 0.25) (layer B.Cu) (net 23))
 (segment (start 123.07498 62.07498) (end 121.5 60.5) (width 0.25) (layer B.Cu) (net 23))
 (segment (start 121.5 60.5) (end 121.5 51.50434) (width 0.25) (layer B.Cu) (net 23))
 (segment (start 121.5 51.50434) (end 124.50434 48.5) (width 0.25) (layer B.Cu) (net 23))
 (segment (start 124.50434 48.5) (end 127 48.5) (width 0.25) (layer B.Cu) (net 23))
 (via (at 125.75 68) (size 0.8) (drill 0.4) (layers F.Cu B.Cu) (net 24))
 (via (at 125.75 65) (size 0.8) (drill 0.4) (layers F.Cu B.Cu) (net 25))
 (segment (start 124.35 65) (end 124.35 66.35) (width 0.25) (layer B.Cu) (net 26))
 (segment (start 124.35 66.35) (end 124.5 66.5) (width 0.25) (layer B.Cu) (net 26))
 (segment (start 124.5 66.5) (end 126.5 66.5) (width 0.25) (layer B.Cu) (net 26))
 (segment (start 126.5 66.5) (end 128.5 64.5) (width 0.25) (layer B.Cu) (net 26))
 (segment (start 128.5 64.5) (end 131.25 64.5) (width 0.25) (layer B.Cu) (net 26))
 (segment (start 131.25 64.5) (end 131.25 64.5) (width 0.25) (layer B.Cu) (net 26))
 (via (at 131.25 64.5) (size 0.8) (drill 0.4) (layers F.Cu B.Cu) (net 26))
 (segment (start 131.15 64.4) (end 131.25 64.5) (width 0.25) (layer F.Cu) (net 26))
 (segment (start 129.85 64.4) (end 131.15 64.4) (width 0.25) (layer F.Cu) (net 26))
 (segment (start 131 45) (end 131 42.75) (width 0.25) (layer F.Cu) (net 26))
 (segment (start 131 42.75) (end 131 42.75) (width 0.25) (layer F.Cu) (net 26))
 (via (at 131 42.75) (size 0.8) (drill 0.4) (layers F.Cu B.Cu) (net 26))
 (segment (start 134.5 46.25) (end 131 42.75) (width 0.25) (layer B.Cu) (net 26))
 (segment (start 132.75 49) (end 134.5 47.25) (width 0.25) (layer B.Cu) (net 26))
 (segment (start 123.52499 64.17499) (end 123.52499 61.8114) (width 0.25) (layer B.Cu) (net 26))
 (segment (start 124.35 65) (end 123.52499 64.17499) (width 0.25) (layer B.Cu) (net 26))
 (segment (start 134.5 47.25) (end 134.5 46.25) (width 0.25) (layer B.Cu) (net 26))
 (segment (start 123.52499 61.8114) (end 122 60.28641) (width 0.25) (layer B.Cu) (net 26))
 (segment (start 122 60.28641) (end 122 51.64075) (width 0.25) (layer B.Cu) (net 26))
 (segment (start 122 51.64075) (end 124.64075 49) (width 0.25) (layer B.Cu) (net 26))
 (segment (start 124.64075 49) (end 132.75 49) (width 0.25) (layer B.Cu) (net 26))
 (via (at 125.75 62) (size 0.8) (drill 0.4) (layers F.Cu B.Cu) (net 27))
 (via (at 131.25 63.5) (size 0.8) (drill 0.4) (layers F.Cu B.Cu) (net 28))
 (segment (start 124.35 62) (end 124.35 62.85) (width 0.25) (layer B.Cu) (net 28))
 (segment (start 125 63.5) (end 131.25 63.5) (width 0.25) (layer B.Cu) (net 28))
 (segment (start 124.35 62.85) (end 125 63.5) (width 0.25) (layer B.Cu) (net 28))
 (segment (start 131.15 63.6) (end 131.25 63.5) (width 0.25) (layer F.Cu) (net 28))
 (segment (start 129.85 63.6) (end 131.15 63.6) (width 0.25) (layer F.Cu) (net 28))
 (segment (start 133 45) (end 133 42.75) (width 0.25) (layer F.Cu) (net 28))
 (segment (start 133 42.75) (end 133 42.75) (width 0.25) (layer F.Cu) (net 28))
 (via (at 133 42.75) (size 0.8) (drill 0.4) (layers F.Cu B.Cu) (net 28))
 (segment (start 122.5 60.15) (end 122.5 51.77716) (width 0.25) (layer B.Cu) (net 28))
 (segment (start 124.35 62) (end 122.5 60.15) (width 0.25) (layer B.Cu) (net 28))
 (segment (start 124.77716 49.5) (end 133 49.5) (width 0.25) (layer B.Cu) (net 28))
 (segment (start 135 44.75) (end 133 42.75) (width 0.25) (layer B.Cu) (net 28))
 (segment (start 122.5 51.77716) (end 124.77716 49.5) (width 0.25) (layer B.Cu) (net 28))
 (segment (start 133 49.5) (end 135 47.5) (width 0.25) (layer B.Cu) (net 28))
 (segment (start 135 47.5) (end 135 44.75) (width 0.25) (layer B.Cu) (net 28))
 (via (at 131.25 62.5) (size 0.8) (drill 0.4) (layers F.Cu B.Cu) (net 29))
 (segment (start 124.35 59.85) (end 125 60.5) (width 0.25) (layer B.Cu) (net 29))
 (segment (start 124.35 59) (end 124.35 59.85) (width 0.25) (layer B.Cu) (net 29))
 (segment (start 125 60.5) (end 126.75 60.5) (width 0.25) (layer B.Cu) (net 29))
 (segment (start 126.75 60.5) (end 128.75 62.5) (width 0.25) (layer B.Cu) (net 29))
 (segment (start 128.75 62.5) (end 131.25 62.5) (width 0.25) (layer B.Cu) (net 29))
 (segment (start 130.95 62.8) (end 131.25 62.5) (width 0.25) (layer F.Cu) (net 29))
 (segment (start 129.85 62.8) (end 130.95 62.8) (width 0.25) (layer F.Cu) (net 29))
 (segment (start 123 45) (end 123 42.75) (width 0.25) (layer F.Cu) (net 29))
 (segment (start 123 42.75) (end 123 42.75) (width 0.25) (layer F.Cu) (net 29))
 (segment (start 124.35 59) (end 123 57.65) (width 0.25) (layer B.Cu) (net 29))
 (segment (start 123 52.5) (end 123 52.25) (width 0.25) (layer B.Cu) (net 29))
 (segment (start 123 57.65) (end 123 52.5) (width 0.25) (layer B.Cu) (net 29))
 (segment (start 124 46.75) (end 123 45.75) (width 0.25) (layer B.Cu) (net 29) (status 1000000))
 (segment (start 123 45.75) (end 123 42.75) (width 0.25) (layer B.Cu) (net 29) (status 1000000))
 (segment (start 125.75 46.75) (end 124 46.75) (width 0.25) (layer B.Cu) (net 29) (status 1000000))
 (segment (start 126 46.5) (end 125.75 46.75) (width 0.25) (layer B.Cu) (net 29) (status 1000000))
 (segment (start 126 40.38641) (end 126 46.5) (width 0.25) (layer B.Cu) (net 29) (status 1000000))
 (segment (start 126.88641 39.5) (end 126 40.38641) (width 0.25) (layer B.Cu) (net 29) (status 1000000))
 (segment (start 135.5 41.5) (end 133.5 39.5) (width 0.25) (layer B.Cu) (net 29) (status 1000000))
 (segment (start 133.5 39.5) (end 126.88641 39.5) (width 0.25) (layer B.Cu) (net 29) (status 1000000))
 (segment (start 135.5 47.75) (end 135.5 41.5) (width 0.25) (layer B.Cu) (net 29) (status 1000000))
 (segment (start 133.25 50) (end 135.5 47.75) (width 0.25) (layer B.Cu) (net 29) (status 1000000))
 (segment (start 124.91357 50) (end 133.25 50) (width 0.25) (layer B.Cu) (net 29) (status 1000000))
 (segment (start 123 52.5) (end 123 51.91357) (width 0.25) (layer B.Cu) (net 29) (status 1000000))
 (segment (start 123 51.91357) (end 124.91357 50) (width 0.25) (layer B.Cu) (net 29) (status 1000000))
 (via (at 123 42.75) (size 0.8) (drill 0.4) (layers F.Cu B.Cu) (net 29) (status 1000000))
 (via (at 125.75 59) (size 0.8) (drill 0.4) (layers F.Cu B.Cu) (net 30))
 (via (at 125.75 56) (size 0.8) (drill 0.4) (layers F.Cu B.Cu) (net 31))
 (segment (start 125 45) (end 125 43.75) (width 0.25) (layer F.Cu) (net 32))
 (segment (start 125 43.75) (end 125 42.75) (width 0.25) (layer F.Cu) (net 32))
 (segment (start 125 42.75) (end 125 42.75) (width 0.25) (layer F.Cu) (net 32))
 (via (at 125 42.75) (size 0.8) (drill 0.4) (layers F.Cu B.Cu) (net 32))
 (segment (start 123.52499 55.17499) (end 123.52499 52.02499) (width 0.25) (layer B.Cu) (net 32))
 (segment (start 124.35 56) (end 123.52499 55.17499) (width 0.25) (layer B.Cu) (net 32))
 (segment (start 124.99999 50.54999) (end 133.45001 50.54999) (width 0.25) (layer B.Cu) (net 32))
 (segment (start 123.52499 52.02499) (end 124.99999 50.54999) (width 0.25) (layer B.Cu) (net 32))
 (segment (start 133.45001 50.54999) (end 136 48) (width 0.25) (layer B.Cu) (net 32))
 (segment (start 136 48) (end 136 41.25) (width 0.25) (layer B.Cu) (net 32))
 (segment (start 136 41.25) (end 133.75 39) (width 0.25) (layer B.Cu) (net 32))
 (segment (start 133.75 39) (end 126.75 39) (width 0.25) (layer B.Cu) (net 32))
 (segment (start 125 40.75) (end 125 42.75) (width 0.25) (layer B.Cu) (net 32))
 (segment (start 126.75 39) (end 125 40.75) (width 0.25) (layer B.Cu) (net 32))
 (segment (start 121 29) (end 121 30.75) (width 0.25) (layer F.Cu) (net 33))
 (segment (start 124.35 53) (end 124.35 51.9) (width 0.25) (layer B.Cu) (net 33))
 (segment (start 124.35 51.9) (end 125.25 51) (width 0.25) (layer B.Cu) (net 33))
 (segment (start 125.25 51) (end 133.75 51) (width 0.25) (layer B.Cu) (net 33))
 (segment (start 133.75 51) (end 136.5 48.25) (width 0.25) (layer B.Cu) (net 33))
 (segment (start 136.5 48.25) (end 136.5 32.25) (width 0.25) (layer B.Cu) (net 33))
 (segment (start 136.5 32.25) (end 135.25 31) (width 0.25) (layer B.Cu) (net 33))
 (segment (start 135.25 31) (end 121 31) (width 0.25) (layer B.Cu) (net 33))
 (segment (start 121 30.75) (end 121 30.75) (width 0.25) (layer F.Cu) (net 33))
 (via (at 121 30.75) (size 0.8) (drill 0.4) (layers F.Cu B.Cu) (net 33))
 (via (at 125.75 53) (size 0.8) (drill 0.4) (layers F.Cu B.Cu) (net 34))
 (via (at 118.75 57.75) (size 0.8) (drill 0.4) (layers F.Cu B.Cu) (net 35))
 (segment (start 125 29) (end 125 32) (width 0.25) (layer F.Cu) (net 35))
 (segment (start 125 32) (end 125 32) (width 0.25) (layer F.Cu) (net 35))
 (via (at 125 32) (size 0.8) (drill 0.4) (layers F.Cu B.Cu) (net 35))
 (segment (start 118.85 57.85) (end 118.75 57.75) (width 0.25) (layer F.Cu) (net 35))
 (segment (start 118.85 58.8) (end 118.85 57.85) (width 0.25) (layer F.Cu) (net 35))
 (via (at 120 59.5) (size 0.8) (drill 0.4) (layers F.Cu B.Cu) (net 38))
 (segment (start 131 29) (end 131 32) (width 0.25) (layer F.Cu) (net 38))
 (segment (start 131 31.75) (end 131 32) (width 0.25) (layer F.Cu) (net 38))
 (segment (start 131 32) (end 131 31.75) (width 0.25) (layer F.Cu) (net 38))
 (via (at 131 32) (size 0.8) (drill 0.4) (layers F.Cu B.Cu) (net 38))
 (segment (start 119.9 59.6) (end 120 59.5) (width 0.25) (layer F.Cu) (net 38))
 (segment (start 118.85 59.6) (end 119.9 59.6) (width 0.25) (layer F.Cu) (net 38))
 (segment (start 120 59.5) (end 121.04999 58.45001) (width 0.25) (layer B.Cu) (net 38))
 (segment (start 121.04999 41.95001) (end 131 32) (width 0.25) (layer B.Cu) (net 38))
 (segment (start 121.04999 58.45001) (end 121.04999 41.95001) (width 0.25) (layer B.Cu) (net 38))
 (via (at 120 60.5) (size 0.8) (drill 0.4) (layers F.Cu B.Cu) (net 37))
 (segment (start 129 29) (end 129 32) (width 0.25) (layer F.Cu) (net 37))
 (segment (start 129 32) (end 129 32) (width 0.25) (layer F.Cu) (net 37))
 (via (at 129 32) (size 0.8) (drill 0.4) (layers F.Cu B.Cu) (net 37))
 (segment (start 119.9 60.4) (end 120 60.5) (width 0.25) (layer F.Cu) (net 37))
 (segment (start 118.85 60.4) (end 119.9 60.4) (width 0.25) (layer F.Cu) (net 37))
 (via (at 118.75 62.25) (size 0.8) (drill 0.4) (layers F.Cu B.Cu) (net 36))
 (segment (start 127 29) (end 127 32) (width 0.25) (layer F.Cu) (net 36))
 (segment (start 127 32) (end 127 32) (width 0.25) (layer F.Cu) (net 36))
 (via (at 127 32) (size 0.8) (drill 0.4) (layers F.Cu B.Cu) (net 36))
 (segment (start 118.85 62.15) (end 118.75 62.25) (width 0.25) (layer F.Cu) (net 36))
 (segment (start 118.85 61.2) (end 118.85 62.15) (width 0.25) (layer F.Cu) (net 36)))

